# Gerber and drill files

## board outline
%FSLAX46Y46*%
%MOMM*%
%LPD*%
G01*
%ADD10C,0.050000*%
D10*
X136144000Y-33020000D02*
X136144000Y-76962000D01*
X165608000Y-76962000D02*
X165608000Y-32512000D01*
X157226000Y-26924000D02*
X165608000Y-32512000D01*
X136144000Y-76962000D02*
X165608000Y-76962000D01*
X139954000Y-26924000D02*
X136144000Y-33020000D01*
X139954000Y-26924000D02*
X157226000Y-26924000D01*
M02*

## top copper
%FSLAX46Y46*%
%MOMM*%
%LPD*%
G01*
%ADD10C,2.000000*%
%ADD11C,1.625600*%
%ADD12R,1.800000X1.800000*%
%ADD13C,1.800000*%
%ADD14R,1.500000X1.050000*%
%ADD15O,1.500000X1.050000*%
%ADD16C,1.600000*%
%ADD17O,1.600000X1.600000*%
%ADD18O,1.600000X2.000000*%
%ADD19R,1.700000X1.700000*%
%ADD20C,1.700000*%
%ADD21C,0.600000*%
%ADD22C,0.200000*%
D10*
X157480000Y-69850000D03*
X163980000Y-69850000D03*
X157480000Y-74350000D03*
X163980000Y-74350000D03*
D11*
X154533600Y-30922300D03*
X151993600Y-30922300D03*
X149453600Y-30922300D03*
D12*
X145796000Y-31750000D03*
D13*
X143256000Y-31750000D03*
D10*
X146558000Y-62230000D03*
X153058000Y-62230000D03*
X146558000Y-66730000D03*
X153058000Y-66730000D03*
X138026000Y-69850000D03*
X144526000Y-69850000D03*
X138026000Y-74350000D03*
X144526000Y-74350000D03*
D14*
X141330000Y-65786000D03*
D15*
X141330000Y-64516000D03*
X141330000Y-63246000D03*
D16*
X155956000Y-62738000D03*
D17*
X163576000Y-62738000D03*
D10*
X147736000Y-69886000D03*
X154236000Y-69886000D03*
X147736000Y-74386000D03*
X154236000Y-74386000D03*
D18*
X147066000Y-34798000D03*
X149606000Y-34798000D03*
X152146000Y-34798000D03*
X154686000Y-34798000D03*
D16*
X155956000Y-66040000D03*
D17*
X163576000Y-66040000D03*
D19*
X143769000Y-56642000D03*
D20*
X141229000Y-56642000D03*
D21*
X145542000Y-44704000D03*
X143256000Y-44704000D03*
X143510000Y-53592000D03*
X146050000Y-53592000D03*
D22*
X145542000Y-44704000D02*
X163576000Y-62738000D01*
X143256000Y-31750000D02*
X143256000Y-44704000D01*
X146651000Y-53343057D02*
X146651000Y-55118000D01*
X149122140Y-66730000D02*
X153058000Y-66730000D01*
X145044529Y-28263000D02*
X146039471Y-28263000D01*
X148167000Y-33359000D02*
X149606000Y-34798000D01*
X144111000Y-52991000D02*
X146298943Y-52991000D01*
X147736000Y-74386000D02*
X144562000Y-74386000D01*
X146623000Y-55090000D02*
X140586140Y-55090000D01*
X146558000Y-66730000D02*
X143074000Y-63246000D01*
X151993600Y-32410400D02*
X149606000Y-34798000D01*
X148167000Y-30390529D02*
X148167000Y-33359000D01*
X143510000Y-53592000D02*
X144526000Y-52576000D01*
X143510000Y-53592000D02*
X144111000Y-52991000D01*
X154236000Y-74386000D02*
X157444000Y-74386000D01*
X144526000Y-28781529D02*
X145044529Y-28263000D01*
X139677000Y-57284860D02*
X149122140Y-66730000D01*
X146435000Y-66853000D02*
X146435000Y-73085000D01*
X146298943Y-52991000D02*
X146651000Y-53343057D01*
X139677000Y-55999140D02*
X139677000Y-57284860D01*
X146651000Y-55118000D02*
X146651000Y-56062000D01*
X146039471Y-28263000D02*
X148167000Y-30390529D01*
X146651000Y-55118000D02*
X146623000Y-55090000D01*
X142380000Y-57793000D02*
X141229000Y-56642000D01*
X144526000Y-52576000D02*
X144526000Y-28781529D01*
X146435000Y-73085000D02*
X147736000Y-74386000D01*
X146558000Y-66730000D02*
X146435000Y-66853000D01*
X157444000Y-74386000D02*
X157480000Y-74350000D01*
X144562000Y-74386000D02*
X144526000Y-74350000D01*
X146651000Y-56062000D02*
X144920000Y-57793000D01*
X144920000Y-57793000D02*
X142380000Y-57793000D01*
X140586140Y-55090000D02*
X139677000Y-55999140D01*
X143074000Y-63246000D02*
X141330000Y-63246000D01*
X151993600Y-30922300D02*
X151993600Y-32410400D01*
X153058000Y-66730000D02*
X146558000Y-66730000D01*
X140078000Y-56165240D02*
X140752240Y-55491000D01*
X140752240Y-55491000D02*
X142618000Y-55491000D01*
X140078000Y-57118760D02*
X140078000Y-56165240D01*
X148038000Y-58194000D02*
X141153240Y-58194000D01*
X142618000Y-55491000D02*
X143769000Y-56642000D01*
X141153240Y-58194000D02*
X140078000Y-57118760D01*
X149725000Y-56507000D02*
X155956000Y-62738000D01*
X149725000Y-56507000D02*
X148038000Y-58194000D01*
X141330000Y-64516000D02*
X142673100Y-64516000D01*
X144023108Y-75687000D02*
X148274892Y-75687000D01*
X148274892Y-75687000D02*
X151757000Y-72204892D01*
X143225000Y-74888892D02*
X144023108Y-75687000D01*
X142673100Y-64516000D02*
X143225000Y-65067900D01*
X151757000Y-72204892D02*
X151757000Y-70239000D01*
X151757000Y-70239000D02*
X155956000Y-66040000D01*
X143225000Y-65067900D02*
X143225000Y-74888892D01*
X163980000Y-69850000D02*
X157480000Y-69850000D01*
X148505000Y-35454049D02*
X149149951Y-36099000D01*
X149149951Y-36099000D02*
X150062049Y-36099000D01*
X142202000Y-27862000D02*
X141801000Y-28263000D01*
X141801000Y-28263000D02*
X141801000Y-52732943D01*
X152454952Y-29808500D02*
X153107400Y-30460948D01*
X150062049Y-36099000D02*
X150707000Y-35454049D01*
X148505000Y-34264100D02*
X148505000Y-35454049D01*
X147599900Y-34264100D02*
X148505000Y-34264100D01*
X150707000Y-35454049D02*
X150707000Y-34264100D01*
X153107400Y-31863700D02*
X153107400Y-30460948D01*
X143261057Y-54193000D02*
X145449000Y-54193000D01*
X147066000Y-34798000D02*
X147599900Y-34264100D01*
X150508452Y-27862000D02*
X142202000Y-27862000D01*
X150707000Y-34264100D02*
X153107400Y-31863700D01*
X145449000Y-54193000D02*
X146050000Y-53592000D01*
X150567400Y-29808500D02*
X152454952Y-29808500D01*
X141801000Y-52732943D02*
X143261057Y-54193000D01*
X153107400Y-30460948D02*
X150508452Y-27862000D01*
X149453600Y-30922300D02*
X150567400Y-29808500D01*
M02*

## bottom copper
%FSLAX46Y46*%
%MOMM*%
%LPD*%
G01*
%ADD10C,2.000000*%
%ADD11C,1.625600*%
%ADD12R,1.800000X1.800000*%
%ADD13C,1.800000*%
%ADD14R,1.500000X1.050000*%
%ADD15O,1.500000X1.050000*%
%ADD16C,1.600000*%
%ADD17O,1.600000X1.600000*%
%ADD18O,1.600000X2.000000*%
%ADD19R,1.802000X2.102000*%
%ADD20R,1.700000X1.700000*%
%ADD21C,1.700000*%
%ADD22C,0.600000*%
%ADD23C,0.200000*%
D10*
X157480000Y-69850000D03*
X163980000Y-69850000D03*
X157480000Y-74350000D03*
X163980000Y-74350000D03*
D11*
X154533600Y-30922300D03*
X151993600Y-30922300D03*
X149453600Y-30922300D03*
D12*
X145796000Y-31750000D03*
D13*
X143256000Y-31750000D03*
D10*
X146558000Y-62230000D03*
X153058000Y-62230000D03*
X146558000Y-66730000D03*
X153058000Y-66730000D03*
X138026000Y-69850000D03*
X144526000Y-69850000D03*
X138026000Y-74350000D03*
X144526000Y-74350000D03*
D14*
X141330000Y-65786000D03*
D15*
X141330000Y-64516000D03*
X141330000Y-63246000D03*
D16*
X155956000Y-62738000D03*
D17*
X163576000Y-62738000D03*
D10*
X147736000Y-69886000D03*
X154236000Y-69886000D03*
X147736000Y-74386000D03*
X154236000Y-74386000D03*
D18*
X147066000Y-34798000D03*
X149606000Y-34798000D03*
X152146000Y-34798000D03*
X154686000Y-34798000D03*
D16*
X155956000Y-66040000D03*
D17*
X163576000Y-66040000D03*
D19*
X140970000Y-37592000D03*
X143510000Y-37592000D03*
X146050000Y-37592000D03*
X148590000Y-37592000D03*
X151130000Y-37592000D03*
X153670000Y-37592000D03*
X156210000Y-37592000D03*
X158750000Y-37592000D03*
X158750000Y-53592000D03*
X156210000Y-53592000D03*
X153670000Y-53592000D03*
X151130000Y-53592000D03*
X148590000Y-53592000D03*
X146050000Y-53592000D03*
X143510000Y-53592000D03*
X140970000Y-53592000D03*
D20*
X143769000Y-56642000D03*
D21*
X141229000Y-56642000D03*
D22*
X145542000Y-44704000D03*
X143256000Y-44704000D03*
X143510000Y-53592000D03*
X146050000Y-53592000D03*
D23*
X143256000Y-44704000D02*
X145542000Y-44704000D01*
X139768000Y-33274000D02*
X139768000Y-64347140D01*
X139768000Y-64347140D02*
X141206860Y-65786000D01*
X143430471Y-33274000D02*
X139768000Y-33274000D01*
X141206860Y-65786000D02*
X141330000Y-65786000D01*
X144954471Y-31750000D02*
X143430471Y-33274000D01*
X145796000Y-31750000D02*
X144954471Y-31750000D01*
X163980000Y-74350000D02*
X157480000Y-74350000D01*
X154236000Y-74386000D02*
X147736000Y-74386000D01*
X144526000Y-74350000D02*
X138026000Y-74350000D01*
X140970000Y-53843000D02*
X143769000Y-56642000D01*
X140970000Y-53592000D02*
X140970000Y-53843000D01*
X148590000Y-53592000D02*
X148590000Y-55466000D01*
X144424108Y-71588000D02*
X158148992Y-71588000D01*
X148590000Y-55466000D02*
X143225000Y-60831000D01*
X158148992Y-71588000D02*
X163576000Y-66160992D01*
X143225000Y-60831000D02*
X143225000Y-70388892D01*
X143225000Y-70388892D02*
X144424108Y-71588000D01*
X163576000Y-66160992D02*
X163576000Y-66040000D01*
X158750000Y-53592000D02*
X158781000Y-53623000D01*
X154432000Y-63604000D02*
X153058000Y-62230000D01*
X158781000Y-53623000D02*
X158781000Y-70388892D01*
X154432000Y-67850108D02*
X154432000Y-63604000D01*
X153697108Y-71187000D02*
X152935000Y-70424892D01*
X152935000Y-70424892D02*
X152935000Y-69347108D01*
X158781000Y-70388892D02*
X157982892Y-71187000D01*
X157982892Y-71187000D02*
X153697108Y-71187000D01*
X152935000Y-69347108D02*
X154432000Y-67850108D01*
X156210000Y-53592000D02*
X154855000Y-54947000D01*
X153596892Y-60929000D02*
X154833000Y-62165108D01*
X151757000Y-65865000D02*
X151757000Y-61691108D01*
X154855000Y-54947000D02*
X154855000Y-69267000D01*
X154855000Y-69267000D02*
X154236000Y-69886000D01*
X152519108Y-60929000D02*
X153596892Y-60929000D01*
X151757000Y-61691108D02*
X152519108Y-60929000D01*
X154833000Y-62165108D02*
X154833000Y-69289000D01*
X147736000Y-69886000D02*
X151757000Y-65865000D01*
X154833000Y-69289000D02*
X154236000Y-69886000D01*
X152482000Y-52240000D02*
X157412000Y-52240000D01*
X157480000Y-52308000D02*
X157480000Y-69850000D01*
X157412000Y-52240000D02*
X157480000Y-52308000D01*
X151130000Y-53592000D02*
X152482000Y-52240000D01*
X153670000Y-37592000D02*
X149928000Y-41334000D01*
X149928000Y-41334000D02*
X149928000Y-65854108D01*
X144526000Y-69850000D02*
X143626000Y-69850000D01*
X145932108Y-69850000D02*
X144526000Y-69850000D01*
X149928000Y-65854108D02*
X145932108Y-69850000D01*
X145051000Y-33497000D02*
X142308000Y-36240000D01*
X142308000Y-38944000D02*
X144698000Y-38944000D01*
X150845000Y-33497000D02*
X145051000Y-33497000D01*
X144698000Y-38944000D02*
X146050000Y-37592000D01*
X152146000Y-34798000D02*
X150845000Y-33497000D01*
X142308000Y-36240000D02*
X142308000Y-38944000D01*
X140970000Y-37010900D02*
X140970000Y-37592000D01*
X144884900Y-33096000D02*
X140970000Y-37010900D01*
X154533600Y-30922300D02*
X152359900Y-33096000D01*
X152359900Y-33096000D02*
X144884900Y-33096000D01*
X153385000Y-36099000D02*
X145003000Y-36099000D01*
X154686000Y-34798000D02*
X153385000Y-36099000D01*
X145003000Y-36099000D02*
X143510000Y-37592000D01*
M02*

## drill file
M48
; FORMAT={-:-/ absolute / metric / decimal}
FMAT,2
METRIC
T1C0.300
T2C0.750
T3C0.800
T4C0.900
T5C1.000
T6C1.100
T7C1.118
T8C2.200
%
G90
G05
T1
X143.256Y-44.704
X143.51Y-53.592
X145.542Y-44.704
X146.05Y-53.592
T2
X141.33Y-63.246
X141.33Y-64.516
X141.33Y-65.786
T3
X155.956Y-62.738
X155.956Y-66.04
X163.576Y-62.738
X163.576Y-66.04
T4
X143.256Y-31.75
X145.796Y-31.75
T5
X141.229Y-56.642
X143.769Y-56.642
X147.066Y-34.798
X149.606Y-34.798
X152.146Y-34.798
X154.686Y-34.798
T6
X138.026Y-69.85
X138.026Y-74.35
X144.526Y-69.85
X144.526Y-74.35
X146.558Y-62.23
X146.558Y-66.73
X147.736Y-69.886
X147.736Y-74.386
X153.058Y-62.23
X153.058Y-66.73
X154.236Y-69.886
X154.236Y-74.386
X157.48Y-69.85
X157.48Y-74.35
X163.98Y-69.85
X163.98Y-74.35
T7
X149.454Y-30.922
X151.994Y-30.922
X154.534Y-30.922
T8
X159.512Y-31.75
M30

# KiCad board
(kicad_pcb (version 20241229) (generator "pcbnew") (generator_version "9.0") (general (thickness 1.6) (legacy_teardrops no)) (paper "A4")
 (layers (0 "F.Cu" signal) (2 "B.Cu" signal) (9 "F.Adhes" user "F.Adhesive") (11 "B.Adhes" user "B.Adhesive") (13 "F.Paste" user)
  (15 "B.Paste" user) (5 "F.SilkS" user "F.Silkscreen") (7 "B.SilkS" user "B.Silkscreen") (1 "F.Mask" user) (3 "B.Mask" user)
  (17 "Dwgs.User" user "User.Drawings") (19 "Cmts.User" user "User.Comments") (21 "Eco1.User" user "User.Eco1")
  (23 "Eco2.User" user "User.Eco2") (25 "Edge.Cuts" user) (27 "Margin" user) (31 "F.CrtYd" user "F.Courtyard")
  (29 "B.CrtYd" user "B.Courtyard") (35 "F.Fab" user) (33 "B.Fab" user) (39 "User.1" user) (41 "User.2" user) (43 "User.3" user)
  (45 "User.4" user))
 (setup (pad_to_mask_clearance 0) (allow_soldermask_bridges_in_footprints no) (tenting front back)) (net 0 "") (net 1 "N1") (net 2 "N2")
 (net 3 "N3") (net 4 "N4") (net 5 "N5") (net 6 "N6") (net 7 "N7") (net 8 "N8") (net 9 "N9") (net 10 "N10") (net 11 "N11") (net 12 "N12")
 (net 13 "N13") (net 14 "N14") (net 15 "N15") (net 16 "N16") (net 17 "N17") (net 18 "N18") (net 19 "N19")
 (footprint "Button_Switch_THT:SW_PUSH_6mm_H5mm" (layer "F.Cu") (at 157.48 69.85)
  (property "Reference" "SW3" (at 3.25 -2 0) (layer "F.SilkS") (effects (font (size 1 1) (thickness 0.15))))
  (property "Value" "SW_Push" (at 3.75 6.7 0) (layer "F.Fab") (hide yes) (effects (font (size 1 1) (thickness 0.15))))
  (pad "1" thru_hole circle (at 0 0 90) (size 2 2) (drill 1.1) (layers "*.Cu" "*.Mask") (remove_unused_layers no) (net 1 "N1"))
  (pad "1" thru_hole circle (at 6.5 0 90) (size 2 2) (drill 1.1) (layers "*.Cu" "*.Mask") (remove_unused_layers no) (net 1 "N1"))
  (pad "2" thru_hole circle (at 0 4.5 90) (size 2 2) (drill 1.1) (layers "*.Cu" "*.Mask") (remove_unused_layers no) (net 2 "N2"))
  (pad "2" thru_hole circle (at 6.5 4.5 90) (size 2 2) (drill 1.1) (layers "*.Cu" "*.Mask") (remove_unused_layers no) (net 2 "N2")))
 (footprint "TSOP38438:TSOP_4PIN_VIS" (layer "F.Cu") (at 154.5336 30.9223 180)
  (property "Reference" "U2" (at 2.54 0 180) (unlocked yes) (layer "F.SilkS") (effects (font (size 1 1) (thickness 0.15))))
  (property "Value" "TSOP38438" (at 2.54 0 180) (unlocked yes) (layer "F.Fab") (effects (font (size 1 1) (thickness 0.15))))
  (pad "1" thru_hole circle (at 0 0 180) (size 1.6256 1.6256) (drill 1.1176) (layers "*.Cu" "*.Mask") (remove_unused_layers no) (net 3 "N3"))
  (pad "2" thru_hole circle (at 2.54 0 180) (size 1.6256 1.6256) (drill 1.1176) (layers "*.Cu" "*.Mask") (remove_unused_layers no)
   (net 2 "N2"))
  (pad "3" thru_hole circle (at 5.08 0 180) (size 1.6256 1.6256) (drill 1.1176) (layers "*.Cu" "*.Mask") (remove_unused_layers no)
   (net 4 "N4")))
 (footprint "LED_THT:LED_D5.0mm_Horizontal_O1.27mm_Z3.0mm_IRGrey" (layer "F.Cu") (at 145.796 31.75 180)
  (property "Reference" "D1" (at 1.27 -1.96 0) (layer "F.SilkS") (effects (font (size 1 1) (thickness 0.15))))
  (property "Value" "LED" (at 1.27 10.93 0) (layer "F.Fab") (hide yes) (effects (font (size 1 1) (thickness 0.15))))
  (pad "1" thru_hole rect (at 0 0 180) (size 1.8 1.8) (drill 0.9) (layers "*.Cu" "*.Mask") (remove_unused_layers no) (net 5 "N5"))
  (pad "2" thru_hole circle (at 2.54 0 180) (size 1.8 1.8) (drill 0.9) (layers "*.Cu" "*.Mask") (remove_unused_layers no) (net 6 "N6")))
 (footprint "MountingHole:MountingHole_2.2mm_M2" (layer "F.Cu") (at 159.512 31.75)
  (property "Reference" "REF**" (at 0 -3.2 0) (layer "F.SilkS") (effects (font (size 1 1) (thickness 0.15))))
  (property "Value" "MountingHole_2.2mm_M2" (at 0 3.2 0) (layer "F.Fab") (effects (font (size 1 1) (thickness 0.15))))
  (pad "" np_thru_hole circle (at 0 0) (size 2.2 2.2) (drill 2.2) (layers "*.Cu" "*.Mask")))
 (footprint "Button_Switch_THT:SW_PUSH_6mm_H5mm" (layer "F.Cu") (at 146.558 62.23)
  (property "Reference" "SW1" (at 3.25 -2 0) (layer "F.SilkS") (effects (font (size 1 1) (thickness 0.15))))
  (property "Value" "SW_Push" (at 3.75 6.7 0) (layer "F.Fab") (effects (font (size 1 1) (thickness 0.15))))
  (pad "1" thru_hole circle (at 0 0 90) (size 2 2) (drill 1.1) (layers "*.Cu" "*.Mask") (remove_unused_layers no) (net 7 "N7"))
  (pad "1" thru_hole circle (at 6.5 0 90) (size 2 2) (drill 1.1) (layers "*.Cu" "*.Mask") (remove_unused_layers no) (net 7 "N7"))
  (pad "2" thru_hole circle (at 0 4.5 90) (size 2 2) (drill 1.1) (layers "*.Cu" "*.Mask") (remove_unused_layers no) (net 2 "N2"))
  (pad "2" thru_hole circle (at 6.5 4.5 90) (size 2 2) (drill 1.1) (layers "*.Cu" "*.Mask") (remove_unused_layers no) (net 2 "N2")))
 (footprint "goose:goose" (layer "F.Cu") (at 154.94 45.466)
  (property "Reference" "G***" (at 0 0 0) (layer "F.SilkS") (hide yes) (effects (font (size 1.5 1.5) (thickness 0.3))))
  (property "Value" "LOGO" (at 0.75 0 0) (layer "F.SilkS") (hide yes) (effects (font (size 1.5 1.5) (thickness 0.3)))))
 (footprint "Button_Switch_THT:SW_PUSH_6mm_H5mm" (layer "F.Cu") (at 138.026 69.85)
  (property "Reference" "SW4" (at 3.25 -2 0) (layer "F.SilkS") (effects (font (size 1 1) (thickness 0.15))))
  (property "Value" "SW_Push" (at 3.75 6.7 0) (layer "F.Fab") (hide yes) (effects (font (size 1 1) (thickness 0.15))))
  (pad "1" thru_hole circle (at 0 0 90) (size 2 2) (drill 1.1) (layers "*.Cu" "*.Mask") (remove_unused_layers no) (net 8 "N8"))
  (pad "1" thru_hole circle (at 6.5 0 90) (size 2 2) (drill 1.1) (layers "*.Cu" "*.Mask") (remove_unused_layers no) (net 8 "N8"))
  (pad "2" thru_hole circle (at 0 4.5 90) (size 2 2) (drill 1.1) (layers "*.Cu" "*.Mask") (remove_unused_layers no) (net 2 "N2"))
  (pad "2" thru_hole circle (at 6.5 4.5 90) (size 2 2) (drill 1.1) (layers "*.Cu" "*.Mask") (remove_unused_layers no) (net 2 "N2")))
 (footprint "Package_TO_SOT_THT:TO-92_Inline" (layer "F.Cu") (at 141.33 65.786 90)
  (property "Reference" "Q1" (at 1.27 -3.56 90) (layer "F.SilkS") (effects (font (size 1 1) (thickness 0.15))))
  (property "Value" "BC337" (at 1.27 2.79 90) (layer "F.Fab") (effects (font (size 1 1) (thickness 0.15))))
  (pad "1" thru_hole rect (at 0 0 90) (size 1.05 1.5) (drill 0.75) (layers "*.Cu" "*.Mask") (remove_unused_layers no) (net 5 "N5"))
  (pad "2" thru_hole oval (at 1.27 0 90) (size 1.05 1.5) (drill 0.75) (layers "*.Cu" "*.Mask") (remove_unused_layers no) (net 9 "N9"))
  (pad "3" thru_hole oval (at 2.54 0 90) (size 1.05 1.5) (drill 0.75) (layers "*.Cu" "*.Mask") (remove_unused_layers no) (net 2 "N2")))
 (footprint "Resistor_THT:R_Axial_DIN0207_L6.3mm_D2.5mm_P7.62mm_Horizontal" (layer "F.Cu") (at 155.956 62.738)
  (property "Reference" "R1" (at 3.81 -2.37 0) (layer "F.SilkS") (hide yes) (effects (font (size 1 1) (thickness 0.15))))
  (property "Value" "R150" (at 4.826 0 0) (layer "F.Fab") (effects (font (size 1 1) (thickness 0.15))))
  (pad "1" thru_hole circle (at 0 0) (size 1.6 1.6) (drill 0.8) (layers "*.Cu" "*.Mask") (remove_unused_layers no) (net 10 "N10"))
  (pad "2" thru_hole oval (at 7.62 0) (size 1.6 1.6) (drill 0.8) (layers "*.Cu" "*.Mask") (remove_unused_layers no) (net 6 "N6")))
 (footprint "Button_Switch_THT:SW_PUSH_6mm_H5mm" (layer "F.Cu") (at 147.736 69.886)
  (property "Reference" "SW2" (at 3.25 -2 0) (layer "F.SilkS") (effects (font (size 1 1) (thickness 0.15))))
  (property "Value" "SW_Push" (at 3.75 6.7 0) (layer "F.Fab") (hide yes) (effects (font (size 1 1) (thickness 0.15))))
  (pad "1" thru_hole circle (at 0 0 90) (size 2 2) (drill 1.1) (layers "*.Cu" "*.Mask") (remove_unused_layers no) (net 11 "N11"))
  (pad "1" thru_hole circle (at 6.5 0 90) (size 2 2) (drill 1.1) (layers "*.Cu" "*.Mask") (remove_unused_layers no) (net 11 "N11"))
  (pad "2" thru_hole circle (at 0 4.5 90) (size 2 2) (drill 1.1) (layers "*.Cu" "*.Mask") (remove_unused_layers no) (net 2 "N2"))
  (pad "2" thru_hole circle (at 6.5 4.5 90) (size 2 2) (drill 1.1) (layers "*.Cu" "*.Mask") (remove_unused_layers no) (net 2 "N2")))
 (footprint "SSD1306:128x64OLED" (layer "F.Cu") (at 150.686 45.398)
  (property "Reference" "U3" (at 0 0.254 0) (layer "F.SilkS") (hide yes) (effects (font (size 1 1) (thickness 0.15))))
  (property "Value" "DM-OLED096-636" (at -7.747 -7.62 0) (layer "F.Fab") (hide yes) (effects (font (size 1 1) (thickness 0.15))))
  (pad "1" thru_hole oval (at -3.62 -10.6 90) (size 2 1.6) (drill 1) (layers "*.Cu" "*.Mask") (remove_unused_layers no) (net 4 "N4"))
  (pad "2" thru_hole oval (at -1.08 -10.6 90) (size 2 1.6) (drill 1) (layers "*.Cu" "*.Mask") (remove_unused_layers no) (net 2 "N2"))
  (pad "3" thru_hole oval (at 1.46 -10.6 90) (size 2 1.6) (drill 1) (layers "*.Cu" "*.Mask") (remove_unused_layers no) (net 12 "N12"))
  (pad "4" thru_hole oval (at 4 -10.6 90) (size 2 1.6) (drill 1) (layers "*.Cu" "*.Mask") (remove_unused_layers no) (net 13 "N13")))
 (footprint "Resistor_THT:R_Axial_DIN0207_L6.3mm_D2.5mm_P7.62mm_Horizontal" (layer "F.Cu") (at 155.956 66.04)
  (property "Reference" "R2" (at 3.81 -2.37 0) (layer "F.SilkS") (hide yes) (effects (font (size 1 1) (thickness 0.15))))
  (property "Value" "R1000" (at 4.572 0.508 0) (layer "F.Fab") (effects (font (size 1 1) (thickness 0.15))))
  (pad "1" thru_hole circle (at 0 0) (size 1.6 1.6) (drill 0.8) (layers "*.Cu" "*.Mask") (remove_unused_layers no) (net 9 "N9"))
  (pad "2" thru_hole oval (at 7.62 0) (size 1.6 1.6) (drill 0.8) (layers "*.Cu" "*.Mask") (remove_unused_layers no) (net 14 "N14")))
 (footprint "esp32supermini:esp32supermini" (layer "B.Cu") (at 149.86 45.592 -90)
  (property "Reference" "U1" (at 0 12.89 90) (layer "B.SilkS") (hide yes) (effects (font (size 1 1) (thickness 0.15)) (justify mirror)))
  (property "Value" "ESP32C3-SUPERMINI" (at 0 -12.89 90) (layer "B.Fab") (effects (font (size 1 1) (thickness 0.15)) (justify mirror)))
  (pad "1" smd rect (at -8 8.89 270) (size 2.102 1.802) (layers "B.Cu" "B.Mask" "B.Paste") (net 3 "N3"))
  (pad "2" smd rect (at -8 6.35 270) (size 2.102 1.802) (layers "B.Cu" "B.Mask" "B.Paste") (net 13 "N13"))
  (pad "3" smd rect (at -8 3.81 270) (size 2.102 1.802) (layers "B.Cu" "B.Mask" "B.Paste") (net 12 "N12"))
  (pad "4" smd rect (at -8 1.27 270) (size 2.102 1.802) (layers "B.Cu" "B.Mask" "B.Paste") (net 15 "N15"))
  (pad "5" smd rect (at -8 -1.27 270) (size 2.102 1.802) (layers "B.Cu" "B.Mask" "B.Paste") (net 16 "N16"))
  (pad "6" smd rect (at -8 -3.81 270) (size 2.102 1.802) (layers "B.Cu" "B.Mask" "B.Paste") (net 8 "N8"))
  (pad "7" smd rect (at -8 -6.35 270) (size 2.102 1.802) (layers "B.Cu" "B.Mask" "B.Paste") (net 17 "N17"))
  (pad "8" smd rect (at -8 -8.89 270) (size 2.102 1.802) (layers "B.Cu" "B.Mask" "B.Paste") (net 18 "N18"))
  (pad "9" smd rect (at 8 -8.89 270) (size 2.102 1.802) (layers "B.Cu" "B.Mask" "B.Paste") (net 7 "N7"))
  (pad "10" smd rect (at 8 -6.35 270) (size 2.102 1.802) (layers "B.Cu" "B.Mask" "B.Paste") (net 11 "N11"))
  (pad "11" smd rect (at 8 -3.81 270) (size 2.102 1.802) (layers "B.Cu" "B.Mask" "B.Paste") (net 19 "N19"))
  (pad "12" smd rect (at 8 -1.27 270) (size 2.102 1.802) (layers "B.Cu" "B.Mask" "B.Paste") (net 1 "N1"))
  (pad "13" smd rect (at 8 1.27 270) (size 2.102 1.802) (layers "B.Cu" "B.Mask" "B.Paste") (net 14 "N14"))
  (pad "14" smd rect (at 8 3.81 270) (size 2.102 1.802) (layers "B.Cu" "B.Mask" "B.Paste") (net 4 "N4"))
  (pad "15" smd rect (at 8 6.35 270) (size 2.102 1.802) (layers "B.Cu" "B.Mask" "B.Paste") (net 2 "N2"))
  (pad "16" smd rect (at 8 8.89 270) (size 2.102 1.802) (layers "B.Cu" "B.Mask" "B.Paste") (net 10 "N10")))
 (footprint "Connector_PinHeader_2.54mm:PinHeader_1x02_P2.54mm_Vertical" (layer "B.Cu") (at 143.769 56.642 90)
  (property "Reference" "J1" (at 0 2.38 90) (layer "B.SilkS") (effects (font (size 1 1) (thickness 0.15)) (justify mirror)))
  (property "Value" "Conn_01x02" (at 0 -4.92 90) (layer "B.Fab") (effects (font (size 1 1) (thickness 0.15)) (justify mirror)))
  (pad "1" thru_hole rect (at 0 0 90) (size 1.7 1.7) (drill 1) (layers "*.Cu" "*.Mask") (remove_unused_layers no) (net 10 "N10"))
  (pad "2" thru_hole circle (at 0 -2.54 90) (size 1.7 1.7) (drill 1) (layers "*.Cu" "*.Mask") (remove_unused_layers no) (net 2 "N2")))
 (gr_line (start 136.144 33.02) (end 136.144 76.962) (stroke (width 0.05) (type default)) (layer "Edge.Cuts"))
 (gr_line (start 165.608 76.962) (end 165.608 32.512) (stroke (width 0.05) (type default)) (layer "Edge.Cuts"))
 (gr_line (start 157.226 26.924) (end 165.608 32.512) (stroke (width 0.05) (type default)) (layer "Edge.Cuts"))
 (gr_line (start 136.144 76.962) (end 165.608 76.962) (stroke (width 0.05) (type default)) (layer "Edge.Cuts"))
 (gr_line (start 139.954 26.924) (end 136.144 33.02) (stroke (width 0.05) (type default)) (layer "Edge.Cuts"))
 (gr_line (start 139.954 26.924) (end 157.226 26.924) (stroke (width 0.05) (type default)) (layer "Edge.Cuts"))
 (segment (start 145.542 44.704) (end 163.576 62.738) (width 0.2) (layer "F.Cu") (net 6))
 (segment (start 143.256 31.75) (end 143.256 44.704) (width 0.2) (layer "F.Cu") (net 6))
 (via (at 145.542 44.704) (size 0.6) (drill 0.3) (layers "F.Cu" "B.Cu") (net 6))
 (via (at 143.256 44.704) (size 0.6) (drill 0.3) (layers "F.Cu" "B.Cu") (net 6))
 (segment (start 143.256 44.704) (end 145.542 44.704) (width 0.2) (layer "B.Cu") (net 6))
 (segment (start 139.768 33.274) (end 139.768 64.34714) (width 0.2) (layer "B.Cu") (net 5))
 (segment (start 139.768 64.34714) (end 141.20686 65.786) (width 0.2) (layer "B.Cu") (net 5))
 (segment (start 143.430471 33.274) (end 139.768 33.274) (width 0.2) (layer "B.Cu") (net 5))
 (segment (start 141.20686 65.786) (end 141.33 65.786) (width 0.2) (layer "B.Cu") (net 5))
 (segment (start 144.954471 31.75) (end 143.430471 33.274) (width 0.2) (layer "B.Cu") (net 5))
 (segment (start 145.796 31.75) (end 144.954471 31.75) (width 0.2) (layer "B.Cu") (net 5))
 (segment (start 146.651 53.343057) (end 146.651 55.118) (width 0.2) (layer "F.Cu") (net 2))
 (segment (start 149.12214 66.73) (end 153.058 66.73) (width 0.2) (layer "F.Cu") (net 2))
 (segment (start 145.044529 28.263) (end 146.039471 28.263) (width 0.2) (layer "F.Cu") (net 2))
 (segment (start 148.167 33.359) (end 149.606 34.798) (width 0.2) (layer "F.Cu") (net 2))
 (segment (start 144.111 52.991) (end 146.298943 52.991) (width 0.2) (layer "F.Cu") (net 2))
 (segment (start 147.736 74.386) (end 144.562 74.386) (width 0.2) (layer "F.Cu") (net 2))
 (segment (start 146.623 55.09) (end 140.58614 55.09) (width 0.2) (layer "F.Cu") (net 2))
 (segment (start 146.558 66.73) (end 143.074 63.246) (width 0.2) (layer "F.Cu") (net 2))
 (segment (start 151.9936 32.4104) (end 149.606 34.798) (width 0.2) (layer "F.Cu") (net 2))
 (segment (start 148.167 30.390529) (end 148.167 33.359) (width 0.2) (layer "F.Cu") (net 2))
 (segment (start 143.51 53.592) (end 144.526 52.576) (width 0.2) (layer "F.Cu") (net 2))
 (segment (start 143.51 53.592) (end 144.111 52.991) (width 0.2) (layer "F.Cu") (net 2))
 (segment (start 154.236 74.386) (end 157.444 74.386) (width 0.2) (layer "F.Cu") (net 2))
 (segment (start 144.526 28.781529) (end 145.044529 28.263) (width 0.2) (layer "F.Cu") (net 2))
 (segment (start 139.677 57.28486) (end 149.12214 66.73) (width 0.2) (layer "F.Cu") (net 2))
 (segment (start 146.435 66.853) (end 146.435 73.085) (width 0.2) (layer "F.Cu") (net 2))
 (segment (start 146.298943 52.991) (end 146.651 53.343057) (width 0.2) (layer "F.Cu") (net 2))
 (segment (start 139.677 55.99914) (end 139.677 57.28486) (width 0.2) (layer "F.Cu") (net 2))
 (segment (start 146.651 55.118) (end 146.651 56.062) (width 0.2) (layer "F.Cu") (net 2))
 (segment (start 146.039471 28.263) (end 148.167 30.390529) (width 0.2) (layer "F.Cu") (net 2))
 (segment (start 146.651 55.118) (end 146.623 55.09) (width 0.2) (layer "F.Cu") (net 2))
 (segment (start 142.38 57.793) (end 141.229 56.642) (width 0.2) (layer "F.Cu") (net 2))
 (segment (start 144.526 52.576) (end 144.526 28.781529) (width 0.2) (layer "F.Cu") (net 2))
 (segment (start 146.435 73.085) (end 147.736 74.386) (width 0.2) (layer "F.Cu") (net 2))
 (segment (start 146.558 66.73) (end 146.435 66.853) (width 0.2) (layer "F.Cu") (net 2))
 (segment (start 157.444 74.386) (end 157.48 74.35) (width 0.2) (layer "F.Cu") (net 2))
 (segment (start 144.562 74.386) (end 144.526 74.35) (width 0.2) (layer "F.Cu") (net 2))
 (segment (start 146.651 56.062) (end 144.92 57.793) (width 0.2) (layer "F.Cu") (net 2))
 (segment (start 144.92 57.793) (end 142.38 57.793) (width 0.2) (layer "F.Cu") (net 2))
 (segment (start 140.58614 55.09) (end 139.677 55.99914) (width 0.2) (layer "F.Cu") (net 2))
 (segment (start 143.074 63.246) (end 141.33 63.246) (width 0.2) (layer "F.Cu") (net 2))
 (segment (start 151.9936 30.9223) (end 151.9936 32.4104) (width 0.2) (layer "F.Cu") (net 2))
 (segment (start 153.058 66.73) (end 146.558 66.73) (width 0.2) (layer "F.Cu") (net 2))
 (via (at 143.51 53.592) (size 0.6) (drill 0.3) (layers "F.Cu" "B.Cu") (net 2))
 (segment (start 163.98 74.35) (end 157.48 74.35) (width 0.2) (layer "B.Cu") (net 2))
 (segment (start 154.236 74.386) (end 147.736 74.386) (width 0.2) (layer "B.Cu") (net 2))
 (segment (start 144.526 74.35) (end 138.026 74.35) (width 0.2) (layer "B.Cu") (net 2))
 (segment (start 140.078 56.16524) (end 140.75224 55.491) (width 0.2) (layer "F.Cu") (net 10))
 (segment (start 140.75224 55.491) (end 142.618 55.491) (width 0.2) (layer "F.Cu") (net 10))
 (segment (start 140.078 57.11876) (end 140.078 56.16524) (width 0.2) (layer "F.Cu") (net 10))
 (segment (start 148.038 58.194) (end 141.15324 58.194) (width 0.2) (layer "F.Cu") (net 10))
 (segment (start 142.618 55.491) (end 143.769 56.642) (width 0.2) (layer "F.Cu") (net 10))
 (segment (start 141.15324 58.194) (end 140.078 57.11876) (width 0.2) (layer "F.Cu") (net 10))
 (segment (start 149.725 56.507) (end 155.956 62.738) (width 0.2) (layer "F.Cu") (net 10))
 (segment (start 149.725 56.507) (end 148.038 58.194) (width 0.2) (layer "F.Cu") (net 10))
 (segment (start 140.97 53.843) (end 143.769 56.642) (width 0.2) (layer "B.Cu") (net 10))
 (segment (start 140.97 53.592) (end 140.97 53.843) (width 0.2) (layer "B.Cu") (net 10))
 (segment (start 141.33 64.516) (end 142.6731 64.516) (width 0.2) (layer "F.Cu") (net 9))
 (segment (start 144.023108 75.687) (end 148.274892 75.687) (width 0.2) (layer "F.Cu") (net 9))
 (segment (start 148.274892 75.687) (end 151.757 72.204892) (width 0.2) (layer "F.Cu") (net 9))
 (segment (start 143.225 74.888892) (end 144.023108 75.687) (width 0.2) (layer "F.Cu") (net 9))
 (segment (start 142.6731 64.516) (end 143.225 65.0679) (width 0.2) (layer "F.Cu") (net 9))
 (segment (start 151.757 72.204892) (end 151.757 70.239) (width 0.2) (layer "F.Cu") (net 9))
 (segment (start 151.757 70.239) (end 155.956 66.04) (width 0.2) (layer "F.Cu") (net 9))
 (segment (start 143.225 65.0679) (end 143.225 74.888892) (width 0.2) (layer "F.Cu") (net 9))
 (segment (start 148.59 53.592) (end 148.59 55.466) (width 0.2) (layer "B.Cu") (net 14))
 (segment (start 144.424108 71.588) (end 158.148992 71.588) (width 0.2) (layer "B.Cu") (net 14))
 (segment (start 148.59 55.466) (end 143.225 60.831) (width 0.2) (layer "B.Cu") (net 14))
 (segment (start 158.148992 71.588) (end 163.576 66.160992) (width 0.2) (layer "B.Cu") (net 14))
 (segment (start 143.225 60.831) (end 143.225 70.388892) (width 0.2) (layer "B.Cu") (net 14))
 (segment (start 143.225 70.388892) (end 144.424108 71.588) (width 0.2) (layer "B.Cu") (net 14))
 (segment (start 163.576 66.160992) (end 163.576 66.04) (width 0.2) (layer "B.Cu") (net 14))
 (segment (start 158.75 53.592) (end 158.781 53.623) (width 0.2) (layer "B.Cu") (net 7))
 (segment (start 154.432 63.604) (end 153.058 62.23) (width 0.2) (layer "B.Cu") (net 7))
 (segment (start 158.781 53.623) (end 158.781 70.388892) (width 0.2) (layer "B.Cu") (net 7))
 (segment (start 154.432 67.850108) (end 154.432 63.604) (width 0.2) (layer "B.Cu") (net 7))
 (segment (start 153.697108 71.187) (end 152.935 70.424892) (width 0.2) (layer "B.Cu") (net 7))
 (segment (start 152.935 70.424892) (end 152.935 69.347108) (width 0.2) (layer "B.Cu") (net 7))
 (segment (start 158.781 70.388892) (end 157.982892 71.187) (width 0.2) (layer "B.Cu") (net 7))
 (segment (start 157.982892 71.187) (end 153.697108 71.187) (width 0.2) (layer "B.Cu") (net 7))
 (segment (start 152.935 69.347108) (end 154.432 67.850108) (width 0.2) (layer "B.Cu") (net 7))
 (segment (start 156.21 53.592) (end 154.855 54.947) (width 0.2) (layer "B.Cu") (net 11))
 (segment (start 153.596892 60.929) (end 154.833 62.165108) (width 0.2) (layer "B.Cu") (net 11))
 (segment (start 151.757 65.865) (end 151.757 61.691108) (width 0.2) (layer "B.Cu") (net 11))
 (segment (start 154.855 54.947) (end 154.855 69.267) (width 0.2) (layer "B.Cu") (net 11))
 (segment (start 154.855 69.267) (end 154.236 69.886) (width 0.2) (layer "B.Cu") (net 11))
 (segment (start 152.519108 60.929) (end 153.596892 60.929) (width 0.2) (layer "B.Cu") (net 11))
 (segment (start 151.757 61.691108) (end 152.519108 60.929) (width 0.2) (layer "B.Cu") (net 11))
 (segment (start 154.833 62.165108) (end 154.833 69.289) (width 0.2) (layer "B.Cu") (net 11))
 (segment (start 147.736 69.886) (end 151.757 65.865) (width 0.2) (layer "B.Cu") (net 11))
 (segment (start 154.833 69.289) (end 154.236 69.886) (width 0.2) (layer "B.Cu") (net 11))
 (segment (start 163.98 69.85) (end 157.48 69.85) (width 0.2) (layer "F.Cu") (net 1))
 (segment (start 152.482 52.24) (end 157.412 52.24) (width 0.2) (layer "B.Cu") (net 1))
 (segment (start 157.48 52.308) (end 157.48 69.85) (width 0.2) (layer "B.Cu") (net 1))
 (segment (start 157.412 52.24) (end 157.48 52.308) (width 0.2) (layer "B.Cu") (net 1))
 (segment (start 151.13 53.592) (end 152.482 52.24) (width 0.2) (layer "B.Cu") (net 1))
 (segment (start 153.67 37.592) (end 149.928 41.334) (width 0.2) (layer "B.Cu") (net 8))
 (segment (start 149.928 41.334) (end 149.928 65.854108) (width 0.2) (layer "B.Cu") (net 8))
 (segment (start 144.526 69.85) (end 143.626 69.85) (width 0.2) (layer "B.Cu") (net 8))
 (segment (start 145.932108 69.85) (end 144.526 69.85) (width 0.2) (layer "B.Cu") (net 8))
 (segment (start 149.928 65.854108) (end 145.932108 69.85) (width 0.2) (layer "B.Cu") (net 8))
 (segment (start 145.051 33.497) (end 142.308 36.24) (width 0.2) (layer "B.Cu") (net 12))
 (segment (start 142.308 38.944) (end 144.698 38.944) (width 0.2) (layer "B.Cu") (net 12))
 (segment (start 150.845 33.497) (end 145.051 33.497) (width 0.2) (layer "B.Cu") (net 12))
 (segment (start 144.698 38.944) (end 146.05 37.592) (width 0.2) (layer "B.Cu") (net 12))
 (segment (start 152.146 34.798) (end 150.845 33.497) (width 0.2) (layer "B.Cu") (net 12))
 (segment (start 142.308 36.24) (end 142.308 38.944) (width 0.2) (layer "B.Cu") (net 12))
 (segment (start 140.97 37.0109) (end 140.97 37.592) (width 0.2) (layer "B.Cu") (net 3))
 (segment (start 144.8849 33.096) (end 140.97 37.0109) (width 0.2) (layer "B.Cu") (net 3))
 (segment (start 154.5336 30.9223) (end 152.3599 33.096) (width 0.2) (layer "B.Cu") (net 3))
 (segment (start 152.3599 33.096) (end 144.8849 33.096) (width 0.2) (layer "B.Cu") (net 3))
 (segment (start 153.385 36.099) (end 145.003 36.099) (width 0.2) (layer "B.Cu") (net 13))
 (segment (start 154.686 34.798) (end 153.385 36.099) (width 0.2) (layer "B.Cu") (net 13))
 (segment (start 145.003 36.099) (end 143.51 37.592) (width 0.2) (layer "B.Cu") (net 13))
 (segment (start 148.505 35.454049) (end 149.149951 36.099) (width 0.2) (layer "F.Cu") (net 4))
 (segment (start 149.149951 36.099) (end 150.062049 36.099) (width 0.2) (layer "F.Cu") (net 4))
 (segment (start 142.202 27.862) (end 141.801 28.263) (width 0.2) (layer "F.Cu") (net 4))
 (segment (start 141.801 28.263) (end 141.801 52.732943) (width 0.2) (layer "F.Cu") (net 4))
 (segment (start 152.454952 29.8085) (end 153.1074 30.460948) (width 0.2) (layer "F.Cu") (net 4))
 (segment (start 150.062049 36.099) (end 150.707 35.454049) (width 0.2) (layer "F.Cu") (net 4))
 (segment (start 148.505 34.2641) (end 148.505 35.454049) (width 0.2) (layer "F.Cu") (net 4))
 (segment (start 147.5999 34.2641) (end 148.505 34.2641) (width 0.2) (layer "F.Cu") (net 4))
 (segment (start 150.707 35.454049) (end 150.707 34.2641) (width 0.2) (layer "F.Cu") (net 4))
 (segment (start 153.1074 31.8637) (end 153.1074 30.460948) (width 0.2) (layer "F.Cu") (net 4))
 (segment (start 143.261057 54.193) (end 145.449 54.193) (width 0.2) (layer "F.Cu") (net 4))
 (segment (start 147.066 34.798) (end 147.5999 34.2641) (width 0.2) (layer "F.Cu") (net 4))
 (segment (start 150.508452 27.862) (end 142.202 27.862) (width 0.2) (layer "F.Cu") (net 4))
 (segment (start 150.707 34.2641) (end 153.1074 31.8637) (width 0.2) (layer "F.Cu") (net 4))
 (segment (start 145.449 54.193) (end 146.05 53.592) (width 0.2) (layer "F.Cu") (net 4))
 (segment (start 150.5674 29.8085) (end 152.454952 29.8085) (width 0.2) (layer "F.Cu") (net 4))
 (segment (start 141.801 52.732943) (end 143.261057 54.193) (width 0.2) (layer "F.Cu") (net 4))
 (segment (start 153.1074 30.460948) (end 150.508452 27.862) (width 0.2) (layer "F.Cu") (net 4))
 (segment (start 149.4536 30.9223) (end 150.5674 29.8085) (width 0.2) (layer "F.Cu") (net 4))
 (via (at 146.05 53.592) (size 0.6) (drill 0.3) (layers "F.Cu" "B.Cu") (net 4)))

